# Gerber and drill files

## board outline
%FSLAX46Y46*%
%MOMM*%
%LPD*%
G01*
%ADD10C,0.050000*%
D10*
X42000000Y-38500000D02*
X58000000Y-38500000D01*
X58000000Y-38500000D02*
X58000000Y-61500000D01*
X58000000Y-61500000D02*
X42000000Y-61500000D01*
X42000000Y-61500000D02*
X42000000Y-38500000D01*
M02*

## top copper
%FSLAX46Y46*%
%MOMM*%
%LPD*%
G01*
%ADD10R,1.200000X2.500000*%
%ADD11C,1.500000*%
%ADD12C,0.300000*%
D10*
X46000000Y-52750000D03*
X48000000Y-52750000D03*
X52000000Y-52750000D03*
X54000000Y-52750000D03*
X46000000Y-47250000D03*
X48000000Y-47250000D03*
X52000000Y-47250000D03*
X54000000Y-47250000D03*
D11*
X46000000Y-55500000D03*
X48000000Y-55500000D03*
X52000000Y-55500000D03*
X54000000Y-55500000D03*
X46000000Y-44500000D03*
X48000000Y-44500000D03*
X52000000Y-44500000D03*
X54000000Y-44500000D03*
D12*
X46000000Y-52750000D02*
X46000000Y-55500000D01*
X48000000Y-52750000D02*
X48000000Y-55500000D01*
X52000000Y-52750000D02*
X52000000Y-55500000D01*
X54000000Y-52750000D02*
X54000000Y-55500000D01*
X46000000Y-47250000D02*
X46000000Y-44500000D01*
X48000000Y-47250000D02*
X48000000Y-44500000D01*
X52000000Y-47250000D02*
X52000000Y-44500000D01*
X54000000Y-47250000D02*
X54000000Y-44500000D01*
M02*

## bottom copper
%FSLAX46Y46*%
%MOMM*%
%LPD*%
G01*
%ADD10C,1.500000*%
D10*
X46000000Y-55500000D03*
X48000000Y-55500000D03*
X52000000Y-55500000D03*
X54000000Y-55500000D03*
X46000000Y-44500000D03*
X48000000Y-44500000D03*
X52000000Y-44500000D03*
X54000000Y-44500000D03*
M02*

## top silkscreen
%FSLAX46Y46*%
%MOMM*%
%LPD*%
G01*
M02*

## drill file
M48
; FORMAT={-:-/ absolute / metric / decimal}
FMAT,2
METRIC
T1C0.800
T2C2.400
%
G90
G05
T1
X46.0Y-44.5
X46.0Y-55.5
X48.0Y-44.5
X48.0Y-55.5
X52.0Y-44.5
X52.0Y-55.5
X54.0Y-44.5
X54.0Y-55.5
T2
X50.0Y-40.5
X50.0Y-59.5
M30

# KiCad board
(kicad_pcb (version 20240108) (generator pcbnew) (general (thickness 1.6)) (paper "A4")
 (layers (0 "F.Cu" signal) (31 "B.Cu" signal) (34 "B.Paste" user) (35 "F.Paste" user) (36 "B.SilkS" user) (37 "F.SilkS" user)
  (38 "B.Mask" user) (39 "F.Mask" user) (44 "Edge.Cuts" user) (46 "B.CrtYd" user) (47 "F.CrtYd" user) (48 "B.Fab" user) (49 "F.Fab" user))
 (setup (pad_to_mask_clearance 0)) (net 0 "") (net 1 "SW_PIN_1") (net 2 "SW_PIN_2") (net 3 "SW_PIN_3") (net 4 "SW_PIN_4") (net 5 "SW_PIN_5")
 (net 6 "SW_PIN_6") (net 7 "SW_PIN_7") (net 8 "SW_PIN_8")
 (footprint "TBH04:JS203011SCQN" (layer "F.Cu") (at 50 50)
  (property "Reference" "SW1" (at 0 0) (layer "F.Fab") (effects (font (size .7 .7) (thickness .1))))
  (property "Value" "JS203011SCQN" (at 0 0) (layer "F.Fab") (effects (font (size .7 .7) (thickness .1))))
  (pad "1" smd rect (at -4 2.75) (size 1.2 2.5) (layers "F.Cu" "F.Paste" "F.Mask") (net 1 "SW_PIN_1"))
  (pad "2" smd rect (at -2 2.75) (size 1.2 2.5) (layers "F.Cu" "F.Paste" "F.Mask") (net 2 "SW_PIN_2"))
  (pad "3" smd rect (at 2 2.75) (size 1.2 2.5) (layers "F.Cu" "F.Paste" "F.Mask") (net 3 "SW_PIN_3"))
  (pad "4" smd rect (at 4 2.75) (size 1.2 2.5) (layers "F.Cu" "F.Paste" "F.Mask") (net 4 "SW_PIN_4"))
  (pad "5" smd rect (at -4 -2.75) (size 1.2 2.5) (layers "F.Cu" "F.Paste" "F.Mask") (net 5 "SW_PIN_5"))
  (pad "6" smd rect (at -2 -2.75) (size 1.2 2.5) (layers "F.Cu" "F.Paste" "F.Mask") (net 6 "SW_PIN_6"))
  (pad "7" smd rect (at 2 -2.75) (size 1.2 2.5) (layers "F.Cu" "F.Paste" "F.Mask") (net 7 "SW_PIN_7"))
  (pad "8" smd rect (at 4 -2.75) (size 1.2 2.5) (layers "F.Cu" "F.Paste" "F.Mask") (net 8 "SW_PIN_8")))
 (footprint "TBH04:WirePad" (layer "F.Cu") (at 46 55.5)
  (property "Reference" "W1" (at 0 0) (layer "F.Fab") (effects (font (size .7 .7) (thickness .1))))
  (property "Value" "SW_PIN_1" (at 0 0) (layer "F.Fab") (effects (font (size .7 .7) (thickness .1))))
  (pad "1" thru_hole circle (at 0 0) (size 1.5 1.5) (drill .8) (layers "*.Cu" "*.Mask") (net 1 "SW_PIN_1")))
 (segment (start 46 52.75) (end 46 55.5) (width .3) (layer "F.Cu") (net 1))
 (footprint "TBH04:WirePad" (layer "F.Cu") (at 48 55.5)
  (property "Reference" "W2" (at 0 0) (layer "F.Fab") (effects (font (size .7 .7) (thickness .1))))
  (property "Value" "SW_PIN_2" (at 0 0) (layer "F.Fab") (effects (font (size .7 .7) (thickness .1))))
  (pad "1" thru_hole circle (at 0 0) (size 1.5 1.5) (drill .8) (layers "*.Cu" "*.Mask") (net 2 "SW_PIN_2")))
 (segment (start 48 52.75) (end 48 55.5) (width .3) (layer "F.Cu") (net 2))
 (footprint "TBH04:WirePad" (layer "F.Cu") (at 52 55.5)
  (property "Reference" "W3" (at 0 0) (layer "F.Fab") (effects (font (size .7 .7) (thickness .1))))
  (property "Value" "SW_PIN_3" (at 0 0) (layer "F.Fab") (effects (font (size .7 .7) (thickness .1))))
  (pad "1" thru_hole circle (at 0 0) (size 1.5 1.5) (drill .8) (layers "*.Cu" "*.Mask") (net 3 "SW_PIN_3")))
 (segment (start 52 52.75) (end 52 55.5) (width .3) (layer "F.Cu") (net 3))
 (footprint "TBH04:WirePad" (layer "F.Cu") (at 54 55.5)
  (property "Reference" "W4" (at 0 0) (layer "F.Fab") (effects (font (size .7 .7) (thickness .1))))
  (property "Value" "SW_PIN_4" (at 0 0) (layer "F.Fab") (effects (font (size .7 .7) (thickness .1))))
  (pad "1" thru_hole circle (at 0 0) (size 1.5 1.5) (drill .8) (layers "*.Cu" "*.Mask") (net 4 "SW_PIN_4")))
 (segment (start 54 52.75) (end 54 55.5) (width .3) (layer "F.Cu") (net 4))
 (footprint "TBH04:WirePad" (layer "F.Cu") (at 46 44.5)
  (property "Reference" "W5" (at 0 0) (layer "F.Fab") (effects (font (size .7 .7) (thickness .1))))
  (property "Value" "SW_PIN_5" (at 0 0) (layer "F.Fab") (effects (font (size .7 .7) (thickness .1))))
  (pad "1" thru_hole circle (at 0 0) (size 1.5 1.5) (drill .8) (layers "*.Cu" "*.Mask") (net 5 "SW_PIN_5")))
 (segment (start 46 47.25) (end 46 44.5) (width .3) (layer "F.Cu") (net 5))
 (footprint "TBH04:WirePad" (layer "F.Cu") (at 48 44.5)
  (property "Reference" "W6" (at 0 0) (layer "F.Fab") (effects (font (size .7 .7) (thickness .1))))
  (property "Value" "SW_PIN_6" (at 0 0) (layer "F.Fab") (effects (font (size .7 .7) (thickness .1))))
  (pad "1" thru_hole circle (at 0 0) (size 1.5 1.5) (drill .8) (layers "*.Cu" "*.Mask") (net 6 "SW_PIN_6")))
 (segment (start 48 47.25) (end 48 44.5) (width .3) (layer "F.Cu") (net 6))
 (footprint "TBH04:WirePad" (layer "F.Cu") (at 52 44.5)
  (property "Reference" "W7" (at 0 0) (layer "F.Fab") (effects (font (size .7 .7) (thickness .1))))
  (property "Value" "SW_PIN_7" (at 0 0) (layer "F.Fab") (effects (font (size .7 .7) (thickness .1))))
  (pad "1" thru_hole circle (at 0 0) (size 1.5 1.5) (drill .8) (layers "*.Cu" "*.Mask") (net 7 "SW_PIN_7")))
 (segment (start 52 47.25) (end 52 44.5) (width .3) (layer "F.Cu") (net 7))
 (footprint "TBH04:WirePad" (layer "F.Cu") (at 54 44.5)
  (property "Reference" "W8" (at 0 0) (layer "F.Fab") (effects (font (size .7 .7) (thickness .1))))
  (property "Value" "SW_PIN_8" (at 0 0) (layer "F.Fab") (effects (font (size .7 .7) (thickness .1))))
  (pad "1" thru_hole circle (at 0 0) (size 1.5 1.5) (drill .8) (layers "*.Cu" "*.Mask") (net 8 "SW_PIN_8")))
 (segment (start 54 47.25) (end 54 44.5) (width .3) (layer "F.Cu") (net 8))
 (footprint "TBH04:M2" (layer "F.Cu") (at 50 40.5)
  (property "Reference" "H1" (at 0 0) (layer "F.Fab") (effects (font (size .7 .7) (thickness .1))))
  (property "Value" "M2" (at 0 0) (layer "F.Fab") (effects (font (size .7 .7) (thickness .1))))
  (pad "" np_thru_hole circle (at 0 0) (size 2.4 2.4) (drill 2.4) (layers "*.Cu" "*.Mask")))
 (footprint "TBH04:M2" (layer "F.Cu") (at 50 59.5)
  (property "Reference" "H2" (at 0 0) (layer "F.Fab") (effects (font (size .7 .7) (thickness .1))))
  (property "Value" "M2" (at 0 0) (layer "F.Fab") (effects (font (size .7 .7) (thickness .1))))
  (pad "" np_thru_hole circle (at 0 0) (size 2.4 2.4) (drill 2.4) (layers "*.Cu" "*.Mask")))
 (gr_line (start 42 38.5) (end 58 38.5) (stroke (width .05) (type default)) (layer "Edge.Cuts"))
 (gr_line (start 58 38.5) (end 58 61.5) (stroke (width .05) (type default)) (layer "Edge.Cuts"))
 (gr_line (start 58 61.5) (end 42 61.5) (stroke (width .05) (type default)) (layer "Edge.Cuts"))
 (gr_line (start 42 61.5) (end 42 38.5) (stroke (width .05) (type default)) (layer "Edge.Cuts")))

